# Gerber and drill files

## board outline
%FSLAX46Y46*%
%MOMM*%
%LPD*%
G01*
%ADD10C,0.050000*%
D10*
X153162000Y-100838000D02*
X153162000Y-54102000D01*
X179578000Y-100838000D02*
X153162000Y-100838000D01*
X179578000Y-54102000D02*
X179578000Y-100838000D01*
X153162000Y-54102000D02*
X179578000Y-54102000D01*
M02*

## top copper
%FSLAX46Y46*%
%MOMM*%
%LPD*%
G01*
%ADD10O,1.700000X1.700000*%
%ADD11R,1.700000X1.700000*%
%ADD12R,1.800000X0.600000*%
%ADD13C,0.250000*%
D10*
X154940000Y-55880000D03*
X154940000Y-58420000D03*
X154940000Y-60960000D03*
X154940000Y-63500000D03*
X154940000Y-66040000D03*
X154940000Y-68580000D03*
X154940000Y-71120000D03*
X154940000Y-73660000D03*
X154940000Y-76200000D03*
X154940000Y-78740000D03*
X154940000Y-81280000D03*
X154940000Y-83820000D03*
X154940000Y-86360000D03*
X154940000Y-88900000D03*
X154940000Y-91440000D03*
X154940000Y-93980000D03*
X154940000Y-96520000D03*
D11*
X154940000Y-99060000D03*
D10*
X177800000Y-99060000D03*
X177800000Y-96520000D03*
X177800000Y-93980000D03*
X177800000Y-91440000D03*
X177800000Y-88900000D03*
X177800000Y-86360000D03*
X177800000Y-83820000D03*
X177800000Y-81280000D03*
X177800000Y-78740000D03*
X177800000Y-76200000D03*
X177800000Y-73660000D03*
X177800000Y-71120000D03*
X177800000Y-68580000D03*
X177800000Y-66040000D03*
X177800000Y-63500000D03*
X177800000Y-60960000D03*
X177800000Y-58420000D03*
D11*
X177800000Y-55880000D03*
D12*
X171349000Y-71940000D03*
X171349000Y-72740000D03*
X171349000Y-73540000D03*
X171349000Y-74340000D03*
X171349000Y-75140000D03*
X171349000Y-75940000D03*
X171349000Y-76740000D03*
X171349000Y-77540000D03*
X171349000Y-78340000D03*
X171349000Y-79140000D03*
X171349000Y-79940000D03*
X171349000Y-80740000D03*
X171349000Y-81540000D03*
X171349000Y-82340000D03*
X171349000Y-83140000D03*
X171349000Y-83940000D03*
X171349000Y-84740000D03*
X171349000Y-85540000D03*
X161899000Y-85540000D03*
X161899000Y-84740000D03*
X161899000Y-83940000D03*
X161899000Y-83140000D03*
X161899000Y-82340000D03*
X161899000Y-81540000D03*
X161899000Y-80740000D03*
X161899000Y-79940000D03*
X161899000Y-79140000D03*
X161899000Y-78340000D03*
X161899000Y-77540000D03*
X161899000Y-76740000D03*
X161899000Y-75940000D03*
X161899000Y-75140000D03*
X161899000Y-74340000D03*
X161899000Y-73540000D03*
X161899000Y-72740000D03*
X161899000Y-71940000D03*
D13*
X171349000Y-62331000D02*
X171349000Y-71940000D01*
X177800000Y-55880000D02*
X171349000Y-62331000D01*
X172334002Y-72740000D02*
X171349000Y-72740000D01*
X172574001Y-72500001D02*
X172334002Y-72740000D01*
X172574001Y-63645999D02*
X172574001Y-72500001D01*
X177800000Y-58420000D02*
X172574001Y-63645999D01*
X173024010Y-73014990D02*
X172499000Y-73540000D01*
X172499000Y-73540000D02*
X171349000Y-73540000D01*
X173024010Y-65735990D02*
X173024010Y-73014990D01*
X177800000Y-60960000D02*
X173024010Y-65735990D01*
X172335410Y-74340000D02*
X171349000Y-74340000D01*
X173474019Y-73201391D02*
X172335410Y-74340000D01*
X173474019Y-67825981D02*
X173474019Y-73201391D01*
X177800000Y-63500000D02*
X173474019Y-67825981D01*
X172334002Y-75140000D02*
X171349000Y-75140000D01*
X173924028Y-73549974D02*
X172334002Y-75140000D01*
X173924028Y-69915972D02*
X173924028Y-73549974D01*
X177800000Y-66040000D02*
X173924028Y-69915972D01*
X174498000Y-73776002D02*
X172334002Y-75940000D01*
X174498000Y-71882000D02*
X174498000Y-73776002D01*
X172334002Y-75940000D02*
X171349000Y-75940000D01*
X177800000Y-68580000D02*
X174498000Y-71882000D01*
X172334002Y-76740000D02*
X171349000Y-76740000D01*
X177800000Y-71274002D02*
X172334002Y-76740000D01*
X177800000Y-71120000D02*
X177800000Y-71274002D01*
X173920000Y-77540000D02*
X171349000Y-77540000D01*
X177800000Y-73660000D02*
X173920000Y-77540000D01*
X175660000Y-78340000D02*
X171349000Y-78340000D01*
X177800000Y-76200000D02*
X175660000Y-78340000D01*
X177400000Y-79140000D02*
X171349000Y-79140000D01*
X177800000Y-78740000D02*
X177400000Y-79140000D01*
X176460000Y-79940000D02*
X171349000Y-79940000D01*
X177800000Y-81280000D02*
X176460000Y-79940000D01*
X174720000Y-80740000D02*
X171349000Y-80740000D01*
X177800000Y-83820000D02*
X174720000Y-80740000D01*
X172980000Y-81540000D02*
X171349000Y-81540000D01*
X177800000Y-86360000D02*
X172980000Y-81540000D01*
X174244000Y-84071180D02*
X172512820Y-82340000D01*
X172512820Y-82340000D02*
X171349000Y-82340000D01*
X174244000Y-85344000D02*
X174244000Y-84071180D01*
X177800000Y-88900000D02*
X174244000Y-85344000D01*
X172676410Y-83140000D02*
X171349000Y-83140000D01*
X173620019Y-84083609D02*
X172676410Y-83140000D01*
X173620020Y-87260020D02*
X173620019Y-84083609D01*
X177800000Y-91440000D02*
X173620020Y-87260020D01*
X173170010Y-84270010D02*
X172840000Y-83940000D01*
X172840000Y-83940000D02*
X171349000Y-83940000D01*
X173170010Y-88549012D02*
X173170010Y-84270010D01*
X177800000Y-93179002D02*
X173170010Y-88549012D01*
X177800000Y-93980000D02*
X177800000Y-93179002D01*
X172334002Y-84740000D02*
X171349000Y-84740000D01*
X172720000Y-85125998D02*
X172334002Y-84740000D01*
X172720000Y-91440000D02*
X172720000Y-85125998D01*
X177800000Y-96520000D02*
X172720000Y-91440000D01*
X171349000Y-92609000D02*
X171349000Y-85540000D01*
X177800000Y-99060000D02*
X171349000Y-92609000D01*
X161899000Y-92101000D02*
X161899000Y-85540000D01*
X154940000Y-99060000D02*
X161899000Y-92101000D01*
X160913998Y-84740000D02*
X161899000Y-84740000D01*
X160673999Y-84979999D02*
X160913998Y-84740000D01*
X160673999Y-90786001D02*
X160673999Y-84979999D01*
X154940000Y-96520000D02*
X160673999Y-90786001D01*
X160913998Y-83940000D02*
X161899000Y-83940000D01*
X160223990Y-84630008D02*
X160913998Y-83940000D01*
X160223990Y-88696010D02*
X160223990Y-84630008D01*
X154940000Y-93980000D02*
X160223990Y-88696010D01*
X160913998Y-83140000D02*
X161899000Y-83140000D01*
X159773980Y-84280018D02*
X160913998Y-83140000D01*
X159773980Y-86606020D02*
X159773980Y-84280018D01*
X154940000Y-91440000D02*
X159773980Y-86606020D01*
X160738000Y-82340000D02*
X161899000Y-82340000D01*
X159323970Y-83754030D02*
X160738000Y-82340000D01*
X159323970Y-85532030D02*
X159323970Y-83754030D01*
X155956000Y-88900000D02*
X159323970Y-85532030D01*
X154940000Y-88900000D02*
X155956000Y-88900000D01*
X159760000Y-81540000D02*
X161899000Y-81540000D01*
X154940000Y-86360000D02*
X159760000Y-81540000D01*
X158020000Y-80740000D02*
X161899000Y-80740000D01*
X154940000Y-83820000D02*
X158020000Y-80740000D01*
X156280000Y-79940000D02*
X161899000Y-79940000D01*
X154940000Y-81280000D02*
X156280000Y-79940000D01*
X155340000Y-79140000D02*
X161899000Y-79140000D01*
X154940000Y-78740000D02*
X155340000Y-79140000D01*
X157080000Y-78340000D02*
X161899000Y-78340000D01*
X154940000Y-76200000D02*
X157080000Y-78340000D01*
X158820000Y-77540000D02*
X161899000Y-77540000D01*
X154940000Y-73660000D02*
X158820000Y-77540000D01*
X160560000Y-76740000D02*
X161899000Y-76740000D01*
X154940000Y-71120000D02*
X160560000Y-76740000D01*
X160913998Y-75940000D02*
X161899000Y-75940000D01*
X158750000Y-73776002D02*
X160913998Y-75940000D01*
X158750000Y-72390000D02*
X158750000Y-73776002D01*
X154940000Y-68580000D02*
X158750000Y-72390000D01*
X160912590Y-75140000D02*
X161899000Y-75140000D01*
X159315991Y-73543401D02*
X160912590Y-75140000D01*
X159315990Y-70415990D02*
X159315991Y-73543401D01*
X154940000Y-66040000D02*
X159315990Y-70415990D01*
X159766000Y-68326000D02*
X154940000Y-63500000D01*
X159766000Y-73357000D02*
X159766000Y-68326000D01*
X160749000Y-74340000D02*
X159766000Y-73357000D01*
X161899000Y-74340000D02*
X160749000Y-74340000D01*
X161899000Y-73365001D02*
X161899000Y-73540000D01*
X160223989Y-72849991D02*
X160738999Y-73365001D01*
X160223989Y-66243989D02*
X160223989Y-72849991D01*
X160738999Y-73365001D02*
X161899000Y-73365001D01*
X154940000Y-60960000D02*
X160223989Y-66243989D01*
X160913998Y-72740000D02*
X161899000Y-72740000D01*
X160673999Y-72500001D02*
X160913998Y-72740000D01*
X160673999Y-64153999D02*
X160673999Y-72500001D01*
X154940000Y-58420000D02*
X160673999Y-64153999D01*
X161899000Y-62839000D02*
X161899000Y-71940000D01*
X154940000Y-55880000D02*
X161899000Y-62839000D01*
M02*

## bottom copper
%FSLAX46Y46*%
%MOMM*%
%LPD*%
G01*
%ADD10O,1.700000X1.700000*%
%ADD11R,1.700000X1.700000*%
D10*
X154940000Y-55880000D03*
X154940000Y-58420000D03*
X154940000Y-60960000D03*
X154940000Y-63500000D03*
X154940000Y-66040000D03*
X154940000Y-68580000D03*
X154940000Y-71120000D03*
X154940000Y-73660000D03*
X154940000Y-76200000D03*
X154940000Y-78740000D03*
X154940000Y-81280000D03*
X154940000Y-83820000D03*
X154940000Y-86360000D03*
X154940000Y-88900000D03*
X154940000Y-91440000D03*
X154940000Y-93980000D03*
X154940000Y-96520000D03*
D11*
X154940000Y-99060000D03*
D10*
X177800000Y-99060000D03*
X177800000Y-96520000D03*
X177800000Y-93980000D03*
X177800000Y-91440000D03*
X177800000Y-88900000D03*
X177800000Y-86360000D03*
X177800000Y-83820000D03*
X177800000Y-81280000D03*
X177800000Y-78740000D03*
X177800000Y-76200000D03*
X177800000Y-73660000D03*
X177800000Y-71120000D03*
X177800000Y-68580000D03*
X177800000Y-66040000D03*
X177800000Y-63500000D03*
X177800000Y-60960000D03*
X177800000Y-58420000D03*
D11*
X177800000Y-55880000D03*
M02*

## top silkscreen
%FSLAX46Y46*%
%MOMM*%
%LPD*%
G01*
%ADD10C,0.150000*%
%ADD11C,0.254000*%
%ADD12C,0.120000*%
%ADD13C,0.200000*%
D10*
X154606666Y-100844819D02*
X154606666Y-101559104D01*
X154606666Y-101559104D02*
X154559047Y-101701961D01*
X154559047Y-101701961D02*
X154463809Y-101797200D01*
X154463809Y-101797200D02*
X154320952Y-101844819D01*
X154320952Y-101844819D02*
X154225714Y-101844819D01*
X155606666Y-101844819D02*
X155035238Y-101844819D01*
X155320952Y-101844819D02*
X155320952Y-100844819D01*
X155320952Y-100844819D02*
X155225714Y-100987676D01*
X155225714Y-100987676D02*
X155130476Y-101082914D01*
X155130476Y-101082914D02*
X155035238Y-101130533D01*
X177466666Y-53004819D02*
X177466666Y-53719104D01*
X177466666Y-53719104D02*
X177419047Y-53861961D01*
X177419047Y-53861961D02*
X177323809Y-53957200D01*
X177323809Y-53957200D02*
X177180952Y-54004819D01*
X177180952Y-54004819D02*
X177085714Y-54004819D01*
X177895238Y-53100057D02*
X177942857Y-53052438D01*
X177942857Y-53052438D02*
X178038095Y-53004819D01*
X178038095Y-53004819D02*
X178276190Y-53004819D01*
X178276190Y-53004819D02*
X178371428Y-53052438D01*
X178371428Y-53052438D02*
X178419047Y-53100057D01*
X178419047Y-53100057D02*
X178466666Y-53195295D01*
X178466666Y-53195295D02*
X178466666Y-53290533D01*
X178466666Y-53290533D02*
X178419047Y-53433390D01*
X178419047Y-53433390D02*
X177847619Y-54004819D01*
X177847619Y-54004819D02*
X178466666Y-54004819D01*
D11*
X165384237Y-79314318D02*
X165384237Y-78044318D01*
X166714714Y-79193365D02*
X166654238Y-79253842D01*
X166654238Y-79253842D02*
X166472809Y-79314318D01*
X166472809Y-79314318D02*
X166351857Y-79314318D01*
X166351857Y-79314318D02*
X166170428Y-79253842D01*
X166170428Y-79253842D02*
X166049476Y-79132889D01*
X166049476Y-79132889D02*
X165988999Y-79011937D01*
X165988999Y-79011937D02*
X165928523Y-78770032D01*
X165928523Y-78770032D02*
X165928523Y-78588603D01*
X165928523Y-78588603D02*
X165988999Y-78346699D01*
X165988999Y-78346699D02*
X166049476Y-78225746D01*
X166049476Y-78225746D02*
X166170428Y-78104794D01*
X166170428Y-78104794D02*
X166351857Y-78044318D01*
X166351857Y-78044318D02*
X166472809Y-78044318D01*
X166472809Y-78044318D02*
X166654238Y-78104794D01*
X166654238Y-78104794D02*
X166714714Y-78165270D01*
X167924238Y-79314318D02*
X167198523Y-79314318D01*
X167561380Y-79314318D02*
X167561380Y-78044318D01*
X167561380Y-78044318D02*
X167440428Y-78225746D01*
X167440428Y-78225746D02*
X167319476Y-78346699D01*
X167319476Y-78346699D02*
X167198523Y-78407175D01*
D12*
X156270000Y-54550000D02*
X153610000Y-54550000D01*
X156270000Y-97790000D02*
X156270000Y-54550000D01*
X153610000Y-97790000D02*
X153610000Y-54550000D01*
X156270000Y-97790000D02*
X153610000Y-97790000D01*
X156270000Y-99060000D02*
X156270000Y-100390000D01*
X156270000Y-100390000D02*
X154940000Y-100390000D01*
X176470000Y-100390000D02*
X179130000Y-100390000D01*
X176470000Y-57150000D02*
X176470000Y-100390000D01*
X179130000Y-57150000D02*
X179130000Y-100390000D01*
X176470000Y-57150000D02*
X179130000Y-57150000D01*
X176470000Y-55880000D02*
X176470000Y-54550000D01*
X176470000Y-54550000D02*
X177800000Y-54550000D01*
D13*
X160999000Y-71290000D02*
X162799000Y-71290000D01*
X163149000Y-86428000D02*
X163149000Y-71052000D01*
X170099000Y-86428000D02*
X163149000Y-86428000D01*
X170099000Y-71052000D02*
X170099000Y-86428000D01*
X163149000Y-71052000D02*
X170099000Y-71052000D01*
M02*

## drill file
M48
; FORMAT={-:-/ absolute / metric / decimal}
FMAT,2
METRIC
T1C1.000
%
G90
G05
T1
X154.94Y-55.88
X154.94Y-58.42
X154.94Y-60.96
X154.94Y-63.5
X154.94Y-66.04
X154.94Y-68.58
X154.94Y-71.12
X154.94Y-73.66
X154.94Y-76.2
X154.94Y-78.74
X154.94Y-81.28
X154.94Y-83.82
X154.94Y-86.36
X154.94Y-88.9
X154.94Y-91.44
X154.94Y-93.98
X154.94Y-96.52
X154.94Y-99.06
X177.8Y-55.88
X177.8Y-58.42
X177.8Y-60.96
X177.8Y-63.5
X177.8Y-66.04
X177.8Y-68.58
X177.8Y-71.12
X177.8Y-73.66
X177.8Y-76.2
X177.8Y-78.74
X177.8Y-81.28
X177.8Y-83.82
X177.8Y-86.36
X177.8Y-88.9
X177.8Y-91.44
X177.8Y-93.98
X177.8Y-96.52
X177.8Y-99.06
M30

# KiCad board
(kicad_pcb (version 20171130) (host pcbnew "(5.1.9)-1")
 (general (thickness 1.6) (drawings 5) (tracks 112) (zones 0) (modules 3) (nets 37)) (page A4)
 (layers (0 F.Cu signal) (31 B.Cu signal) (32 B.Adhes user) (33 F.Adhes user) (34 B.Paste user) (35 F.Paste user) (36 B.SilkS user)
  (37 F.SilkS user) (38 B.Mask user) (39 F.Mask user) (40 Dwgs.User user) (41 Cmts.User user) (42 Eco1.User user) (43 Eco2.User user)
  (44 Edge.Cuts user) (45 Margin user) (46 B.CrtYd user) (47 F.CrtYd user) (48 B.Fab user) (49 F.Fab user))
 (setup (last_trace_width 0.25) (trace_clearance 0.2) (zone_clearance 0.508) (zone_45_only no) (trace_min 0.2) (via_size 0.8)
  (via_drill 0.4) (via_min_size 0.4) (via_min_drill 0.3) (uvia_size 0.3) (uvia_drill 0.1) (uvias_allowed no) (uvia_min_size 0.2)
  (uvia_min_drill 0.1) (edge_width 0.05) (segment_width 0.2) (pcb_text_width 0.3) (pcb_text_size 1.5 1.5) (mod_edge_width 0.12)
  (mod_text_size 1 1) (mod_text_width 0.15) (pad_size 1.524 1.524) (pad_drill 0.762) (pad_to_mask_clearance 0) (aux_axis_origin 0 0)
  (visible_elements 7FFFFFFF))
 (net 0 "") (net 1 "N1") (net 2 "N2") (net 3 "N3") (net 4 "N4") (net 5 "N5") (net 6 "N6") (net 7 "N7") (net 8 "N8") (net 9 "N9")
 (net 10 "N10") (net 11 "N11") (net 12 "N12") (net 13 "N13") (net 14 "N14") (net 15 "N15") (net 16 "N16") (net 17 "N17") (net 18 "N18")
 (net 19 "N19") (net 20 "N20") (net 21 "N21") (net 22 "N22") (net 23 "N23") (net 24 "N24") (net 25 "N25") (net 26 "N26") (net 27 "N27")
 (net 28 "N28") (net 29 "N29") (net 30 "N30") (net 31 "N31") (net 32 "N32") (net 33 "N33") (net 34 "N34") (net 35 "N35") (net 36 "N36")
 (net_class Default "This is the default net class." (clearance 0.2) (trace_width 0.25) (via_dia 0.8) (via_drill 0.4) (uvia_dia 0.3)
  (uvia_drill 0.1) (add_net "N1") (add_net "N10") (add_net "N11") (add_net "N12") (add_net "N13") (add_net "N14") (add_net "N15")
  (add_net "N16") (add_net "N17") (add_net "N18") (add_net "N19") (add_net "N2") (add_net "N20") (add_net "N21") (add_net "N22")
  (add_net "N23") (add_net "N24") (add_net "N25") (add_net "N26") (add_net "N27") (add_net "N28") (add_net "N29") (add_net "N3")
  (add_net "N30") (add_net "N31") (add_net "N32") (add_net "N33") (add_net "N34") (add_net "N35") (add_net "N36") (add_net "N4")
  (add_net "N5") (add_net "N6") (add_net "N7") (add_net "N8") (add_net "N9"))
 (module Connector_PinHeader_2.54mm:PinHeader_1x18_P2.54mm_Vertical (layer F.Cu) (at 154.94 99.06 180)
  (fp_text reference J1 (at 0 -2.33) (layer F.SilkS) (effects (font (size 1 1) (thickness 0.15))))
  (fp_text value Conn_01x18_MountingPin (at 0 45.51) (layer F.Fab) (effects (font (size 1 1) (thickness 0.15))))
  (fp_line (start -1.33 44.51) (end 1.33 44.51) (layer F.SilkS) (width 0.12))
  (fp_line (start -1.33 1.27) (end -1.33 44.51) (layer F.SilkS) (width 0.12))
  (fp_line (start 1.33 1.27) (end 1.33 44.51) (layer F.SilkS) (width 0.12))
  (fp_line (start -1.33 1.27) (end 1.33 1.27) (layer F.SilkS) (width 0.12))
  (fp_line (start -1.33 0) (end -1.33 -1.33) (layer F.SilkS) (width 0.12))
  (fp_line (start -1.33 -1.33) (end 0 -1.33) (layer F.SilkS) (width 0.12))
  (pad 18 thru_hole oval (at 0 43.18 180) (size 1.7 1.7) (drill 1) (layers *.Cu *.Mask) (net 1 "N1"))
  (pad 17 thru_hole oval (at 0 40.64 180) (size 1.7 1.7) (drill 1) (layers *.Cu *.Mask) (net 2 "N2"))
  (pad 16 thru_hole oval (at 0 38.1 180) (size 1.7 1.7) (drill 1) (layers *.Cu *.Mask) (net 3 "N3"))
  (pad 15 thru_hole oval (at 0 35.56 180) (size 1.7 1.7) (drill 1) (layers *.Cu *.Mask) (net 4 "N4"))
  (pad 14 thru_hole oval (at 0 33.02 180) (size 1.7 1.7) (drill 1) (layers *.Cu *.Mask) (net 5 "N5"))
  (pad 13 thru_hole oval (at 0 30.48 180) (size 1.7 1.7) (drill 1) (layers *.Cu *.Mask) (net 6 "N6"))
  (pad 12 thru_hole oval (at 0 27.94 180) (size 1.7 1.7) (drill 1) (layers *.Cu *.Mask) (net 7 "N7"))
  (pad 11 thru_hole oval (at 0 25.4 180) (size 1.7 1.7) (drill 1) (layers *.Cu *.Mask) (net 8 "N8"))
  (pad 10 thru_hole oval (at 0 22.86 180) (size 1.7 1.7) (drill 1) (layers *.Cu *.Mask) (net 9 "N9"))
  (pad 9 thru_hole oval (at 0 20.32 180) (size 1.7 1.7) (drill 1) (layers *.Cu *.Mask) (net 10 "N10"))
  (pad 8 thru_hole oval (at 0 17.78 180) (size 1.7 1.7) (drill 1) (layers *.Cu *.Mask) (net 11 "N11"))
  (pad 7 thru_hole oval (at 0 15.24 180) (size 1.7 1.7) (drill 1) (layers *.Cu *.Mask) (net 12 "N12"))
  (pad 6 thru_hole oval (at 0 12.7 180) (size 1.7 1.7) (drill 1) (layers *.Cu *.Mask) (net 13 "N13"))
  (pad 5 thru_hole oval (at 0 10.16 180) (size 1.7 1.7) (drill 1) (layers *.Cu *.Mask) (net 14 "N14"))
  (pad 4 thru_hole oval (at 0 7.62 180) (size 1.7 1.7) (drill 1) (layers *.Cu *.Mask) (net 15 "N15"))
  (pad 3 thru_hole oval (at 0 5.08 180) (size 1.7 1.7) (drill 1) (layers *.Cu *.Mask) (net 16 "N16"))
  (pad 2 thru_hole oval (at 0 2.54 180) (size 1.7 1.7) (drill 1) (layers *.Cu *.Mask) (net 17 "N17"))
  (pad 1 thru_hole rect (at 0 0 180) (size 1.7 1.7) (drill 1) (layers *.Cu *.Mask) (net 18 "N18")))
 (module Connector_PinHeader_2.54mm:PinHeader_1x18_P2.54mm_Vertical (layer F.Cu) (at 177.8 55.88)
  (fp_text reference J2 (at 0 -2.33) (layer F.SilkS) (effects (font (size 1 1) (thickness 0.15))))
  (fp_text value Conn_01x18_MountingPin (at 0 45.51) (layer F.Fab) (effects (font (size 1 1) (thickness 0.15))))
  (fp_line (start -1.33 44.51) (end 1.33 44.51) (layer F.SilkS) (width 0.12))
  (fp_line (start -1.33 1.27) (end -1.33 44.51) (layer F.SilkS) (width 0.12))
  (fp_line (start 1.33 1.27) (end 1.33 44.51) (layer F.SilkS) (width 0.12))
  (fp_line (start -1.33 1.27) (end 1.33 1.27) (layer F.SilkS) (width 0.12))
  (fp_line (start -1.33 0) (end -1.33 -1.33) (layer F.SilkS) (width 0.12))
  (fp_line (start -1.33 -1.33) (end 0 -1.33) (layer F.SilkS) (width 0.12))
  (pad 18 thru_hole oval (at 0 43.18) (size 1.7 1.7) (drill 1) (layers *.Cu *.Mask) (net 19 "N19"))
  (pad 17 thru_hole oval (at 0 40.64) (size 1.7 1.7) (drill 1) (layers *.Cu *.Mask) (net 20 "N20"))
  (pad 16 thru_hole oval (at 0 38.1) (size 1.7 1.7) (drill 1) (layers *.Cu *.Mask) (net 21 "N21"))
  (pad 15 thru_hole oval (at 0 35.56) (size 1.7 1.7) (drill 1) (layers *.Cu *.Mask) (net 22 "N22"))
  (pad 14 thru_hole oval (at 0 33.02) (size 1.7 1.7) (drill 1) (layers *.Cu *.Mask) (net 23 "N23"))
  (pad 13 thru_hole oval (at 0 30.48) (size 1.7 1.7) (drill 1) (layers *.Cu *.Mask) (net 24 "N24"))
  (pad 12 thru_hole oval (at 0 27.94) (size 1.7 1.7) (drill 1) (layers *.Cu *.Mask) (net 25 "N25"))
  (pad 11 thru_hole oval (at 0 25.4) (size 1.7 1.7) (drill 1) (layers *.Cu *.Mask) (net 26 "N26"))
  (pad 10 thru_hole oval (at 0 22.86) (size 1.7 1.7) (drill 1) (layers *.Cu *.Mask) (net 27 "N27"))
  (pad 9 thru_hole oval (at 0 20.32) (size 1.7 1.7) (drill 1) (layers *.Cu *.Mask) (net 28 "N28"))
  (pad 8 thru_hole oval (at 0 17.78) (size 1.7 1.7) (drill 1) (layers *.Cu *.Mask) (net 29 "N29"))
  (pad 7 thru_hole oval (at 0 15.24) (size 1.7 1.7) (drill 1) (layers *.Cu *.Mask) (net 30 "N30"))
  (pad 6 thru_hole oval (at 0 12.7) (size 1.7 1.7) (drill 1) (layers *.Cu *.Mask) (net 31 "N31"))
  (pad 5 thru_hole oval (at 0 10.16) (size 1.7 1.7) (drill 1) (layers *.Cu *.Mask) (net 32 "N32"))
  (pad 4 thru_hole oval (at 0 7.62) (size 1.7 1.7) (drill 1) (layers *.Cu *.Mask) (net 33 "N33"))
  (pad 3 thru_hole oval (at 0 5.08) (size 1.7 1.7) (drill 1) (layers *.Cu *.Mask) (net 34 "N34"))
  (pad 2 thru_hole oval (at 0 2.54) (size 1.7 1.7) (drill 1) (layers *.Cu *.Mask) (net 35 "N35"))
  (pad 1 thru_hole rect (at 0 0) (size 1.7 1.7) (drill 1) (layers *.Cu *.Mask) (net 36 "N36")))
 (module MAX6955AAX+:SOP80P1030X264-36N (layer F.Cu) (at 166.624 78.74)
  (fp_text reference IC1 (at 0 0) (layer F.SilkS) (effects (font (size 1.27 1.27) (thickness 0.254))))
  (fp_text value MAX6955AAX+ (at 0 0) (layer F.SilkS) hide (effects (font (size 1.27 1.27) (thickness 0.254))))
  (fp_line (start -5.625 -7.45) (end -3.825 -7.45) (layer F.SilkS) (width 0.2))
  (fp_line (start -3.475 7.688) (end -3.475 -7.688) (layer F.SilkS) (width 0.2))
  (fp_line (start 3.475 7.688) (end -3.475 7.688) (layer F.SilkS) (width 0.2))
  (fp_line (start 3.475 -7.688) (end 3.475 7.688) (layer F.SilkS) (width 0.2))
  (fp_line (start -3.475 -7.688) (end 3.475 -7.688) (layer F.SilkS) (width 0.2))
  (pad 36 smd rect (at 4.725 -6.8 90) (size 0.6 1.8) (layers F.Cu F.Paste F.Mask) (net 36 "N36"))
  (pad 35 smd rect (at 4.725 -6 90) (size 0.6 1.8) (layers F.Cu F.Paste F.Mask) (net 35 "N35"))
  (pad 34 smd rect (at 4.725 -5.2 90) (size 0.6 1.8) (layers F.Cu F.Paste F.Mask) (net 34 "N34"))
  (pad 33 smd rect (at 4.725 -4.4 90) (size 0.6 1.8) (layers F.Cu F.Paste F.Mask) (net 33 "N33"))
  (pad 32 smd rect (at 4.725 -3.6 90) (size 0.6 1.8) (layers F.Cu F.Paste F.Mask) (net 32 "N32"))
  (pad 31 smd rect (at 4.725 -2.8 90) (size 0.6 1.8) (layers F.Cu F.Paste F.Mask) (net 31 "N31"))
  (pad 30 smd rect (at 4.725 -2 90) (size 0.6 1.8) (layers F.Cu F.Paste F.Mask) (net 30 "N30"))
  (pad 29 smd rect (at 4.725 -1.2 90) (size 0.6 1.8) (layers F.Cu F.Paste F.Mask) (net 29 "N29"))
  (pad 28 smd rect (at 4.725 -0.4 90) (size 0.6 1.8) (layers F.Cu F.Paste F.Mask) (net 28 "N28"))
  (pad 27 smd rect (at 4.725 0.4 90) (size 0.6 1.8) (layers F.Cu F.Paste F.Mask) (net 27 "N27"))
  (pad 26 smd rect (at 4.725 1.2 90) (size 0.6 1.8) (layers F.Cu F.Paste F.Mask) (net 26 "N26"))
  (pad 25 smd rect (at 4.725 2 90) (size 0.6 1.8) (layers F.Cu F.Paste F.Mask) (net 25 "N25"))
  (pad 24 smd rect (at 4.725 2.8 90) (size 0.6 1.8) (layers F.Cu F.Paste F.Mask) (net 24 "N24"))
  (pad 23 smd rect (at 4.725 3.6 90) (size 0.6 1.8) (layers F.Cu F.Paste F.Mask) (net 23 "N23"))
  (pad 22 smd rect (at 4.725 4.4 90) (size 0.6 1.8) (layers F.Cu F.Paste F.Mask) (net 22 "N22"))
  (pad 21 smd rect (at 4.725 5.2 90) (size 0.6 1.8) (layers F.Cu F.Paste F.Mask) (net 21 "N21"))
  (pad 20 smd rect (at 4.725 6 90) (size 0.6 1.8) (layers F.Cu F.Paste F.Mask) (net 20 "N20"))
  (pad 19 smd rect (at 4.725 6.8 90) (size 0.6 1.8) (layers F.Cu F.Paste F.Mask) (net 19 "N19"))
  (pad 18 smd rect (at -4.725 6.8 90) (size 0.6 1.8) (layers F.Cu F.Paste F.Mask) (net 18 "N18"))
  (pad 17 smd rect (at -4.725 6 90) (size 0.6 1.8) (layers F.Cu F.Paste F.Mask) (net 17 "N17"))
  (pad 16 smd rect (at -4.725 5.2 90) (size 0.6 1.8) (layers F.Cu F.Paste F.Mask) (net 16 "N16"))
  (pad 15 smd rect (at -4.725 4.4 90) (size 0.6 1.8) (layers F.Cu F.Paste F.Mask) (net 15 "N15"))
  (pad 14 smd rect (at -4.725 3.6 90) (size 0.6 1.8) (layers F.Cu F.Paste F.Mask) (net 14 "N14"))
  (pad 13 smd rect (at -4.725 2.8 90) (size 0.6 1.8) (layers F.Cu F.Paste F.Mask) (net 13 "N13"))
  (pad 12 smd rect (at -4.725 2 90) (size 0.6 1.8) (layers F.Cu F.Paste F.Mask) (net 12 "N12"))
  (pad 11 smd rect (at -4.725 1.2 90) (size 0.6 1.8) (layers F.Cu F.Paste F.Mask) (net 11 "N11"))
  (pad 10 smd rect (at -4.725 0.4 90) (size 0.6 1.8) (layers F.Cu F.Paste F.Mask) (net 10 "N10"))
  (pad 9 smd rect (at -4.725 -0.4 90) (size 0.6 1.8) (layers F.Cu F.Paste F.Mask) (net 9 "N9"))
  (pad 8 smd rect (at -4.725 -1.2 90) (size 0.6 1.8) (layers F.Cu F.Paste F.Mask) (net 8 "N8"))
  (pad 7 smd rect (at -4.725 -2 90) (size 0.6 1.8) (layers F.Cu F.Paste F.Mask) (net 7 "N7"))
  (pad 6 smd rect (at -4.725 -2.8 90) (size 0.6 1.8) (layers F.Cu F.Paste F.Mask) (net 6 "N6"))
  (pad 5 smd rect (at -4.725 -3.6 90) (size 0.6 1.8) (layers F.Cu F.Paste F.Mask) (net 5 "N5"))
  (pad 4 smd rect (at -4.725 -4.4 90) (size 0.6 1.8) (layers F.Cu F.Paste F.Mask) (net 4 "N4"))
  (pad 3 smd rect (at -4.725 -5.2 90) (size 0.6 1.8) (layers F.Cu F.Paste F.Mask) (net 3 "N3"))
  (pad 2 smd rect (at -4.725 -6 90) (size 0.6 1.8) (layers F.Cu F.Paste F.Mask) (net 2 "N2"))
  (pad 1 smd rect (at -4.725 -6.8 90) (size 0.6 1.8) (layers F.Cu F.Paste F.Mask) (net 1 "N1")))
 (gr_line (start 153.162 100.838) (end 153.162 54.102) (layer Edge.Cuts) (width 0.05))
 (gr_line (start 179.578 100.838) (end 153.162 100.838) (layer Edge.Cuts) (width 0.05))
 (gr_line (start 179.578 54.102) (end 179.578 100.838) (layer Edge.Cuts) (width 0.05))
 (gr_line (start 153.162 54.102) (end 179.578 54.102) (layer Edge.Cuts) (width 0.05))
 (segment (start 171.349 62.331) (end 171.349 71.94) (width 0.25) (layer F.Cu) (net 36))
 (segment (start 177.8 55.88) (end 171.349 62.331) (width 0.25) (layer F.Cu) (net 36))
 (segment (start 172.334002 72.74) (end 171.349 72.74) (width 0.25) (layer F.Cu) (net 35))
 (segment (start 172.574001 72.500001) (end 172.334002 72.74) (width 0.25) (layer F.Cu) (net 35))
 (segment (start 172.574001 63.645999) (end 172.574001 72.500001) (width 0.25) (layer F.Cu) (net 35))
 (segment (start 177.8 58.42) (end 172.574001 63.645999) (width 0.25) (layer F.Cu) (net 35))
 (segment (start 173.02401 73.01499) (end 172.499 73.54) (width 0.25) (layer F.Cu) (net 34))
 (segment (start 172.499 73.54) (end 171.349 73.54) (width 0.25) (layer F.Cu) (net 34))
 (segment (start 173.02401 65.73599) (end 173.02401 73.01499) (width 0.25) (layer F.Cu) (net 34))
 (segment (start 177.8 60.96) (end 173.02401 65.73599) (width 0.25) (layer F.Cu) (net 34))
 (segment (start 172.33541 74.34) (end 171.349 74.34) (width 0.25) (layer F.Cu) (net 33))
 (segment (start 173.474019 73.201391) (end 172.33541 74.34) (width 0.25) (layer F.Cu) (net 33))
 (segment (start 173.474019 67.825981) (end 173.474019 73.201391) (width 0.25) (layer F.Cu) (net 33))
 (segment (start 177.8 63.5) (end 173.474019 67.825981) (width 0.25) (layer F.Cu) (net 33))
 (segment (start 172.334002 75.14) (end 171.349 75.14) (width 0.25) (layer F.Cu) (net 32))
 (segment (start 173.924028 73.549974) (end 172.334002 75.14) (width 0.25) (layer F.Cu) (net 32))
 (segment (start 173.924028 69.915972) (end 173.924028 73.549974) (width 0.25) (layer F.Cu) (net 32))
 (segment (start 177.8 66.04) (end 173.924028 69.915972) (width 0.25) (layer F.Cu) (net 32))
 (segment (start 174.498 73.776002) (end 172.334002 75.94) (width 0.25) (layer F.Cu) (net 31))
 (segment (start 174.498 71.882) (end 174.498 73.776002) (width 0.25) (layer F.Cu) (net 31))
 (segment (start 172.334002 75.94) (end 171.349 75.94) (width 0.25) (layer F.Cu) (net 31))
 (segment (start 177.8 68.58) (end 174.498 71.882) (width 0.25) (layer F.Cu) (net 31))
 (segment (start 172.334002 76.74) (end 171.349 76.74) (width 0.25) (layer F.Cu) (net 30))
 (segment (start 177.8 71.274002) (end 172.334002 76.74) (width 0.25) (layer F.Cu) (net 30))
 (segment (start 177.8 71.12) (end 177.8 71.274002) (width 0.25) (layer F.Cu) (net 30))
 (segment (start 173.92 77.54) (end 171.349 77.54) (width 0.25) (layer F.Cu) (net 29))
 (segment (start 177.8 73.66) (end 173.92 77.54) (width 0.25) (layer F.Cu) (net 29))
 (segment (start 175.66 78.34) (end 171.349 78.34) (width 0.25) (layer F.Cu) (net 28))
 (segment (start 177.8 76.2) (end 175.66 78.34) (width 0.25) (layer F.Cu) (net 28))
 (segment (start 177.4 79.14) (end 171.349 79.14) (width 0.25) (layer F.Cu) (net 27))
 (segment (start 177.8 78.74) (end 177.4 79.14) (width 0.25) (layer F.Cu) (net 27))
 (segment (start 176.46 79.94) (end 171.349 79.94) (width 0.25) (layer F.Cu) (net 26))
 (segment (start 177.8 81.28) (end 176.46 79.94) (width 0.25) (layer F.Cu) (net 26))
 (segment (start 174.72 80.74) (end 171.349 80.74) (width 0.25) (layer F.Cu) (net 25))
 (segment (start 177.8 83.82) (end 174.72 80.74) (width 0.25) (layer F.Cu) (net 25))
 (segment (start 172.98 81.54) (end 171.349 81.54) (width 0.25) (layer F.Cu) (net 24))
 (segment (start 177.8 86.36) (end 172.98 81.54) (width 0.25) (layer F.Cu) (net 24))
 (segment (start 174.244 84.07118) (end 172.51282 82.34) (width 0.25) (layer F.Cu) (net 23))
 (segment (start 172.51282 82.34) (end 171.349 82.34) (width 0.25) (layer F.Cu) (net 23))
 (segment (start 174.244 85.344) (end 174.244 84.07118) (width 0.25) (layer F.Cu) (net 23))
 (segment (start 177.8 88.9) (end 174.244 85.344) (width 0.25) (layer F.Cu) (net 23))
 (segment (start 172.67641 83.14) (end 171.349 83.14) (width 0.25) (layer F.Cu) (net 22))
 (segment (start 173.620019 84.083609) (end 172.67641 83.14) (width 0.25) (layer F.Cu) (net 22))
 (segment (start 173.62002 87.26002) (end 173.620019 84.083609) (width 0.25) (layer F.Cu) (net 22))
 (segment (start 177.8 91.44) (end 173.62002 87.26002) (width 0.25) (layer F.Cu) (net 22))
 (segment (start 173.17001 84.27001) (end 172.84 83.94) (width 0.25) (layer F.Cu) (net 21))
 (segment (start 172.84 83.94) (end 171.349 83.94) (width 0.25) (layer F.Cu) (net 21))
 (segment (start 173.17001 88.549012) (end 173.17001 84.27001) (width 0.25) (layer F.Cu) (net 21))
 (segment (start 177.8 93.179002) (end 173.17001 88.549012) (width 0.25) (layer F.Cu) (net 21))
 (segment (start 177.8 93.98) (end 177.8 93.179002) (width 0.25) (layer F.Cu) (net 21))
 (segment (start 172.334002 84.74) (end 171.349 84.74) (width 0.25) (layer F.Cu) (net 20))
 (segment (start 172.72 85.125998) (end 172.334002 84.74) (width 0.25) (layer F.Cu) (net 20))
 (segment (start 172.72 91.44) (end 172.72 85.125998) (width 0.25) (layer F.Cu) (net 20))
 (segment (start 177.8 96.52) (end 172.72 91.44) (width 0.25) (layer F.Cu) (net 20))
 (segment (start 171.349 92.609) (end 171.349 85.54) (width 0.25) (layer F.Cu) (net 19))
 (segment (start 177.8 99.06) (end 171.349 92.609) (width 0.25) (layer F.Cu) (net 19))
 (segment (start 161.899 92.101) (end 161.899 85.54) (width 0.25) (layer F.Cu) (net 18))
 (segment (start 154.94 99.06) (end 161.899 92.101) (width 0.25) (layer F.Cu) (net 18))
 (segment (start 160.913998 84.74) (end 161.899 84.74) (width 0.25) (layer F.Cu) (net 17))
 (segment (start 160.673999 84.979999) (end 160.913998 84.74) (width 0.25) (layer F.Cu) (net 17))
 (segment (start 160.673999 90.786001) (end 160.673999 84.979999) (width 0.25) (layer F.Cu) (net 17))
 (segment (start 154.94 96.52) (end 160.673999 90.786001) (width 0.25) (layer F.Cu) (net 17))
 (segment (start 160.913998 83.94) (end 161.899 83.94) (width 0.25) (layer F.Cu) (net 16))
 (segment (start 160.22399 84.630008) (end 160.913998 83.94) (width 0.25) (layer F.Cu) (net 16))
 (segment (start 160.22399 88.69601) (end 160.22399 84.630008) (width 0.25) (layer F.Cu) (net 16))
 (segment (start 154.94 93.98) (end 160.22399 88.69601) (width 0.25) (layer F.Cu) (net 16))
 (segment (start 160.913998 83.14) (end 161.899 83.14) (width 0.25) (layer F.Cu) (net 15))
 (segment (start 159.77398 84.280018) (end 160.913998 83.14) (width 0.25) (layer F.Cu) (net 15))
 (segment (start 159.77398 86.60602) (end 159.77398 84.280018) (width 0.25) (layer F.Cu) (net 15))
 (segment (start 154.94 91.44) (end 159.77398 86.60602) (width 0.25) (layer F.Cu) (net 15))
 (segment (start 160.738 82.34) (end 161.899 82.34) (width 0.25) (layer F.Cu) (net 14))
 (segment (start 159.32397 83.75403) (end 160.738 82.34) (width 0.25) (layer F.Cu) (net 14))
 (segment (start 159.32397 85.53203) (end 159.32397 83.75403) (width 0.25) (layer F.Cu) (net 14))
 (segment (start 155.956 88.9) (end 159.32397 85.53203) (width 0.25) (layer F.Cu) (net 14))
 (segment (start 154.94 88.9) (end 155.956 88.9) (width 0.25) (layer F.Cu) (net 14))
 (segment (start 159.76 81.54) (end 161.899 81.54) (width 0.25) (layer F.Cu) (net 13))
 (segment (start 154.94 86.36) (end 159.76 81.54) (width 0.25) (layer F.Cu) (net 13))
 (segment (start 158.02 80.74) (end 161.899 80.74) (width 0.25) (layer F.Cu) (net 12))
 (segment (start 154.94 83.82) (end 158.02 80.74) (width 0.25) (layer F.Cu) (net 12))
 (segment (start 156.28 79.94) (end 161.899 79.94) (width 0.25) (layer F.Cu) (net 11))
 (segment (start 154.94 81.28) (end 156.28 79.94) (width 0.25) (layer F.Cu) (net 11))
 (segment (start 155.34 79.14) (end 161.899 79.14) (width 0.25) (layer F.Cu) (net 10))
 (segment (start 154.94 78.74) (end 155.34 79.14) (width 0.25) (layer F.Cu) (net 10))
 (segment (start 157.08 78.34) (end 161.899 78.34) (width 0.25) (layer F.Cu) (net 9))
 (segment (start 154.94 76.2) (end 157.08 78.34) (width 0.25) (layer F.Cu) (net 9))
 (segment (start 158.82 77.54) (end 161.899 77.54) (width 0.25) (layer F.Cu) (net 8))
 (segment (start 154.94 73.66) (end 158.82 77.54) (width 0.25) (layer F.Cu) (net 8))
 (segment (start 160.56 76.74) (end 161.899 76.74) (width 0.25) (layer F.Cu) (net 7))
 (segment (start 154.94 71.12) (end 160.56 76.74) (width 0.25) (layer F.Cu) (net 7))
 (segment (start 160.913998 75.94) (end 161.899 75.94) (width 0.25) (layer F.Cu) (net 6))
 (segment (start 158.75 73.776002) (end 160.913998 75.94) (width 0.25) (layer F.Cu) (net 6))
 (segment (start 158.75 72.39) (end 158.75 73.776002) (width 0.25) (layer F.Cu) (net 6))
 (segment (start 154.94 68.58) (end 158.75 72.39) (width 0.25) (layer F.Cu) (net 6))
 (segment (start 160.91259 75.14) (end 161.899 75.14) (width 0.25) (layer F.Cu) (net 5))
 (segment (start 159.315991 73.543401) (end 160.91259 75.14) (width 0.25) (layer F.Cu) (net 5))
 (segment (start 159.31599 70.41599) (end 159.315991 73.543401) (width 0.25) (layer F.Cu) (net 5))
 (segment (start 154.94 66.04) (end 159.31599 70.41599) (width 0.25) (layer F.Cu) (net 5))
 (segment (start 159.766 68.326) (end 154.94 63.5) (width 0.25) (layer F.Cu) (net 4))
 (segment (start 159.766 73.357) (end 159.766 68.326) (width 0.25) (layer F.Cu) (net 4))
 (segment (start 160.749 74.34) (end 159.766 73.357) (width 0.25) (layer F.Cu) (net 4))
 (segment (start 161.899 74.34) (end 160.749 74.34) (width 0.25) (layer F.Cu) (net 4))
 (segment (start 161.899 73.365001) (end 161.899 73.54) (width 0.25) (layer F.Cu) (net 3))
 (segment (start 160.223989 72.849991) (end 160.738999 73.365001) (width 0.25) (layer F.Cu) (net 3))
 (segment (start 160.223989 66.243989) (end 160.223989 72.849991) (width 0.25) (layer F.Cu) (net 3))
 (segment (start 160.738999 73.365001) (end 161.899 73.365001) (width 0.25) (layer F.Cu) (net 3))
 (segment (start 154.94 60.96) (end 160.223989 66.243989) (width 0.25) (layer F.Cu) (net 3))
 (segment (start 160.913998 72.74) (end 161.899 72.74) (width 0.25) (layer F.Cu) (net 2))
 (segment (start 160.673999 72.500001) (end 160.913998 72.74) (width 0.25) (layer F.Cu) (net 2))
 (segment (start 160.673999 64.153999) (end 160.673999 72.500001) (width 0.25) (layer F.Cu) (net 2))
 (segment (start 154.94 58.42) (end 160.673999 64.153999) (width 0.25) (layer F.Cu) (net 2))
 (segment (start 161.899 62.839) (end 161.899 71.94) (width 0.25) (layer F.Cu) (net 1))
 (segment (start 154.94 55.88) (end 161.899 62.839) (width 0.25) (layer F.Cu) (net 1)))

